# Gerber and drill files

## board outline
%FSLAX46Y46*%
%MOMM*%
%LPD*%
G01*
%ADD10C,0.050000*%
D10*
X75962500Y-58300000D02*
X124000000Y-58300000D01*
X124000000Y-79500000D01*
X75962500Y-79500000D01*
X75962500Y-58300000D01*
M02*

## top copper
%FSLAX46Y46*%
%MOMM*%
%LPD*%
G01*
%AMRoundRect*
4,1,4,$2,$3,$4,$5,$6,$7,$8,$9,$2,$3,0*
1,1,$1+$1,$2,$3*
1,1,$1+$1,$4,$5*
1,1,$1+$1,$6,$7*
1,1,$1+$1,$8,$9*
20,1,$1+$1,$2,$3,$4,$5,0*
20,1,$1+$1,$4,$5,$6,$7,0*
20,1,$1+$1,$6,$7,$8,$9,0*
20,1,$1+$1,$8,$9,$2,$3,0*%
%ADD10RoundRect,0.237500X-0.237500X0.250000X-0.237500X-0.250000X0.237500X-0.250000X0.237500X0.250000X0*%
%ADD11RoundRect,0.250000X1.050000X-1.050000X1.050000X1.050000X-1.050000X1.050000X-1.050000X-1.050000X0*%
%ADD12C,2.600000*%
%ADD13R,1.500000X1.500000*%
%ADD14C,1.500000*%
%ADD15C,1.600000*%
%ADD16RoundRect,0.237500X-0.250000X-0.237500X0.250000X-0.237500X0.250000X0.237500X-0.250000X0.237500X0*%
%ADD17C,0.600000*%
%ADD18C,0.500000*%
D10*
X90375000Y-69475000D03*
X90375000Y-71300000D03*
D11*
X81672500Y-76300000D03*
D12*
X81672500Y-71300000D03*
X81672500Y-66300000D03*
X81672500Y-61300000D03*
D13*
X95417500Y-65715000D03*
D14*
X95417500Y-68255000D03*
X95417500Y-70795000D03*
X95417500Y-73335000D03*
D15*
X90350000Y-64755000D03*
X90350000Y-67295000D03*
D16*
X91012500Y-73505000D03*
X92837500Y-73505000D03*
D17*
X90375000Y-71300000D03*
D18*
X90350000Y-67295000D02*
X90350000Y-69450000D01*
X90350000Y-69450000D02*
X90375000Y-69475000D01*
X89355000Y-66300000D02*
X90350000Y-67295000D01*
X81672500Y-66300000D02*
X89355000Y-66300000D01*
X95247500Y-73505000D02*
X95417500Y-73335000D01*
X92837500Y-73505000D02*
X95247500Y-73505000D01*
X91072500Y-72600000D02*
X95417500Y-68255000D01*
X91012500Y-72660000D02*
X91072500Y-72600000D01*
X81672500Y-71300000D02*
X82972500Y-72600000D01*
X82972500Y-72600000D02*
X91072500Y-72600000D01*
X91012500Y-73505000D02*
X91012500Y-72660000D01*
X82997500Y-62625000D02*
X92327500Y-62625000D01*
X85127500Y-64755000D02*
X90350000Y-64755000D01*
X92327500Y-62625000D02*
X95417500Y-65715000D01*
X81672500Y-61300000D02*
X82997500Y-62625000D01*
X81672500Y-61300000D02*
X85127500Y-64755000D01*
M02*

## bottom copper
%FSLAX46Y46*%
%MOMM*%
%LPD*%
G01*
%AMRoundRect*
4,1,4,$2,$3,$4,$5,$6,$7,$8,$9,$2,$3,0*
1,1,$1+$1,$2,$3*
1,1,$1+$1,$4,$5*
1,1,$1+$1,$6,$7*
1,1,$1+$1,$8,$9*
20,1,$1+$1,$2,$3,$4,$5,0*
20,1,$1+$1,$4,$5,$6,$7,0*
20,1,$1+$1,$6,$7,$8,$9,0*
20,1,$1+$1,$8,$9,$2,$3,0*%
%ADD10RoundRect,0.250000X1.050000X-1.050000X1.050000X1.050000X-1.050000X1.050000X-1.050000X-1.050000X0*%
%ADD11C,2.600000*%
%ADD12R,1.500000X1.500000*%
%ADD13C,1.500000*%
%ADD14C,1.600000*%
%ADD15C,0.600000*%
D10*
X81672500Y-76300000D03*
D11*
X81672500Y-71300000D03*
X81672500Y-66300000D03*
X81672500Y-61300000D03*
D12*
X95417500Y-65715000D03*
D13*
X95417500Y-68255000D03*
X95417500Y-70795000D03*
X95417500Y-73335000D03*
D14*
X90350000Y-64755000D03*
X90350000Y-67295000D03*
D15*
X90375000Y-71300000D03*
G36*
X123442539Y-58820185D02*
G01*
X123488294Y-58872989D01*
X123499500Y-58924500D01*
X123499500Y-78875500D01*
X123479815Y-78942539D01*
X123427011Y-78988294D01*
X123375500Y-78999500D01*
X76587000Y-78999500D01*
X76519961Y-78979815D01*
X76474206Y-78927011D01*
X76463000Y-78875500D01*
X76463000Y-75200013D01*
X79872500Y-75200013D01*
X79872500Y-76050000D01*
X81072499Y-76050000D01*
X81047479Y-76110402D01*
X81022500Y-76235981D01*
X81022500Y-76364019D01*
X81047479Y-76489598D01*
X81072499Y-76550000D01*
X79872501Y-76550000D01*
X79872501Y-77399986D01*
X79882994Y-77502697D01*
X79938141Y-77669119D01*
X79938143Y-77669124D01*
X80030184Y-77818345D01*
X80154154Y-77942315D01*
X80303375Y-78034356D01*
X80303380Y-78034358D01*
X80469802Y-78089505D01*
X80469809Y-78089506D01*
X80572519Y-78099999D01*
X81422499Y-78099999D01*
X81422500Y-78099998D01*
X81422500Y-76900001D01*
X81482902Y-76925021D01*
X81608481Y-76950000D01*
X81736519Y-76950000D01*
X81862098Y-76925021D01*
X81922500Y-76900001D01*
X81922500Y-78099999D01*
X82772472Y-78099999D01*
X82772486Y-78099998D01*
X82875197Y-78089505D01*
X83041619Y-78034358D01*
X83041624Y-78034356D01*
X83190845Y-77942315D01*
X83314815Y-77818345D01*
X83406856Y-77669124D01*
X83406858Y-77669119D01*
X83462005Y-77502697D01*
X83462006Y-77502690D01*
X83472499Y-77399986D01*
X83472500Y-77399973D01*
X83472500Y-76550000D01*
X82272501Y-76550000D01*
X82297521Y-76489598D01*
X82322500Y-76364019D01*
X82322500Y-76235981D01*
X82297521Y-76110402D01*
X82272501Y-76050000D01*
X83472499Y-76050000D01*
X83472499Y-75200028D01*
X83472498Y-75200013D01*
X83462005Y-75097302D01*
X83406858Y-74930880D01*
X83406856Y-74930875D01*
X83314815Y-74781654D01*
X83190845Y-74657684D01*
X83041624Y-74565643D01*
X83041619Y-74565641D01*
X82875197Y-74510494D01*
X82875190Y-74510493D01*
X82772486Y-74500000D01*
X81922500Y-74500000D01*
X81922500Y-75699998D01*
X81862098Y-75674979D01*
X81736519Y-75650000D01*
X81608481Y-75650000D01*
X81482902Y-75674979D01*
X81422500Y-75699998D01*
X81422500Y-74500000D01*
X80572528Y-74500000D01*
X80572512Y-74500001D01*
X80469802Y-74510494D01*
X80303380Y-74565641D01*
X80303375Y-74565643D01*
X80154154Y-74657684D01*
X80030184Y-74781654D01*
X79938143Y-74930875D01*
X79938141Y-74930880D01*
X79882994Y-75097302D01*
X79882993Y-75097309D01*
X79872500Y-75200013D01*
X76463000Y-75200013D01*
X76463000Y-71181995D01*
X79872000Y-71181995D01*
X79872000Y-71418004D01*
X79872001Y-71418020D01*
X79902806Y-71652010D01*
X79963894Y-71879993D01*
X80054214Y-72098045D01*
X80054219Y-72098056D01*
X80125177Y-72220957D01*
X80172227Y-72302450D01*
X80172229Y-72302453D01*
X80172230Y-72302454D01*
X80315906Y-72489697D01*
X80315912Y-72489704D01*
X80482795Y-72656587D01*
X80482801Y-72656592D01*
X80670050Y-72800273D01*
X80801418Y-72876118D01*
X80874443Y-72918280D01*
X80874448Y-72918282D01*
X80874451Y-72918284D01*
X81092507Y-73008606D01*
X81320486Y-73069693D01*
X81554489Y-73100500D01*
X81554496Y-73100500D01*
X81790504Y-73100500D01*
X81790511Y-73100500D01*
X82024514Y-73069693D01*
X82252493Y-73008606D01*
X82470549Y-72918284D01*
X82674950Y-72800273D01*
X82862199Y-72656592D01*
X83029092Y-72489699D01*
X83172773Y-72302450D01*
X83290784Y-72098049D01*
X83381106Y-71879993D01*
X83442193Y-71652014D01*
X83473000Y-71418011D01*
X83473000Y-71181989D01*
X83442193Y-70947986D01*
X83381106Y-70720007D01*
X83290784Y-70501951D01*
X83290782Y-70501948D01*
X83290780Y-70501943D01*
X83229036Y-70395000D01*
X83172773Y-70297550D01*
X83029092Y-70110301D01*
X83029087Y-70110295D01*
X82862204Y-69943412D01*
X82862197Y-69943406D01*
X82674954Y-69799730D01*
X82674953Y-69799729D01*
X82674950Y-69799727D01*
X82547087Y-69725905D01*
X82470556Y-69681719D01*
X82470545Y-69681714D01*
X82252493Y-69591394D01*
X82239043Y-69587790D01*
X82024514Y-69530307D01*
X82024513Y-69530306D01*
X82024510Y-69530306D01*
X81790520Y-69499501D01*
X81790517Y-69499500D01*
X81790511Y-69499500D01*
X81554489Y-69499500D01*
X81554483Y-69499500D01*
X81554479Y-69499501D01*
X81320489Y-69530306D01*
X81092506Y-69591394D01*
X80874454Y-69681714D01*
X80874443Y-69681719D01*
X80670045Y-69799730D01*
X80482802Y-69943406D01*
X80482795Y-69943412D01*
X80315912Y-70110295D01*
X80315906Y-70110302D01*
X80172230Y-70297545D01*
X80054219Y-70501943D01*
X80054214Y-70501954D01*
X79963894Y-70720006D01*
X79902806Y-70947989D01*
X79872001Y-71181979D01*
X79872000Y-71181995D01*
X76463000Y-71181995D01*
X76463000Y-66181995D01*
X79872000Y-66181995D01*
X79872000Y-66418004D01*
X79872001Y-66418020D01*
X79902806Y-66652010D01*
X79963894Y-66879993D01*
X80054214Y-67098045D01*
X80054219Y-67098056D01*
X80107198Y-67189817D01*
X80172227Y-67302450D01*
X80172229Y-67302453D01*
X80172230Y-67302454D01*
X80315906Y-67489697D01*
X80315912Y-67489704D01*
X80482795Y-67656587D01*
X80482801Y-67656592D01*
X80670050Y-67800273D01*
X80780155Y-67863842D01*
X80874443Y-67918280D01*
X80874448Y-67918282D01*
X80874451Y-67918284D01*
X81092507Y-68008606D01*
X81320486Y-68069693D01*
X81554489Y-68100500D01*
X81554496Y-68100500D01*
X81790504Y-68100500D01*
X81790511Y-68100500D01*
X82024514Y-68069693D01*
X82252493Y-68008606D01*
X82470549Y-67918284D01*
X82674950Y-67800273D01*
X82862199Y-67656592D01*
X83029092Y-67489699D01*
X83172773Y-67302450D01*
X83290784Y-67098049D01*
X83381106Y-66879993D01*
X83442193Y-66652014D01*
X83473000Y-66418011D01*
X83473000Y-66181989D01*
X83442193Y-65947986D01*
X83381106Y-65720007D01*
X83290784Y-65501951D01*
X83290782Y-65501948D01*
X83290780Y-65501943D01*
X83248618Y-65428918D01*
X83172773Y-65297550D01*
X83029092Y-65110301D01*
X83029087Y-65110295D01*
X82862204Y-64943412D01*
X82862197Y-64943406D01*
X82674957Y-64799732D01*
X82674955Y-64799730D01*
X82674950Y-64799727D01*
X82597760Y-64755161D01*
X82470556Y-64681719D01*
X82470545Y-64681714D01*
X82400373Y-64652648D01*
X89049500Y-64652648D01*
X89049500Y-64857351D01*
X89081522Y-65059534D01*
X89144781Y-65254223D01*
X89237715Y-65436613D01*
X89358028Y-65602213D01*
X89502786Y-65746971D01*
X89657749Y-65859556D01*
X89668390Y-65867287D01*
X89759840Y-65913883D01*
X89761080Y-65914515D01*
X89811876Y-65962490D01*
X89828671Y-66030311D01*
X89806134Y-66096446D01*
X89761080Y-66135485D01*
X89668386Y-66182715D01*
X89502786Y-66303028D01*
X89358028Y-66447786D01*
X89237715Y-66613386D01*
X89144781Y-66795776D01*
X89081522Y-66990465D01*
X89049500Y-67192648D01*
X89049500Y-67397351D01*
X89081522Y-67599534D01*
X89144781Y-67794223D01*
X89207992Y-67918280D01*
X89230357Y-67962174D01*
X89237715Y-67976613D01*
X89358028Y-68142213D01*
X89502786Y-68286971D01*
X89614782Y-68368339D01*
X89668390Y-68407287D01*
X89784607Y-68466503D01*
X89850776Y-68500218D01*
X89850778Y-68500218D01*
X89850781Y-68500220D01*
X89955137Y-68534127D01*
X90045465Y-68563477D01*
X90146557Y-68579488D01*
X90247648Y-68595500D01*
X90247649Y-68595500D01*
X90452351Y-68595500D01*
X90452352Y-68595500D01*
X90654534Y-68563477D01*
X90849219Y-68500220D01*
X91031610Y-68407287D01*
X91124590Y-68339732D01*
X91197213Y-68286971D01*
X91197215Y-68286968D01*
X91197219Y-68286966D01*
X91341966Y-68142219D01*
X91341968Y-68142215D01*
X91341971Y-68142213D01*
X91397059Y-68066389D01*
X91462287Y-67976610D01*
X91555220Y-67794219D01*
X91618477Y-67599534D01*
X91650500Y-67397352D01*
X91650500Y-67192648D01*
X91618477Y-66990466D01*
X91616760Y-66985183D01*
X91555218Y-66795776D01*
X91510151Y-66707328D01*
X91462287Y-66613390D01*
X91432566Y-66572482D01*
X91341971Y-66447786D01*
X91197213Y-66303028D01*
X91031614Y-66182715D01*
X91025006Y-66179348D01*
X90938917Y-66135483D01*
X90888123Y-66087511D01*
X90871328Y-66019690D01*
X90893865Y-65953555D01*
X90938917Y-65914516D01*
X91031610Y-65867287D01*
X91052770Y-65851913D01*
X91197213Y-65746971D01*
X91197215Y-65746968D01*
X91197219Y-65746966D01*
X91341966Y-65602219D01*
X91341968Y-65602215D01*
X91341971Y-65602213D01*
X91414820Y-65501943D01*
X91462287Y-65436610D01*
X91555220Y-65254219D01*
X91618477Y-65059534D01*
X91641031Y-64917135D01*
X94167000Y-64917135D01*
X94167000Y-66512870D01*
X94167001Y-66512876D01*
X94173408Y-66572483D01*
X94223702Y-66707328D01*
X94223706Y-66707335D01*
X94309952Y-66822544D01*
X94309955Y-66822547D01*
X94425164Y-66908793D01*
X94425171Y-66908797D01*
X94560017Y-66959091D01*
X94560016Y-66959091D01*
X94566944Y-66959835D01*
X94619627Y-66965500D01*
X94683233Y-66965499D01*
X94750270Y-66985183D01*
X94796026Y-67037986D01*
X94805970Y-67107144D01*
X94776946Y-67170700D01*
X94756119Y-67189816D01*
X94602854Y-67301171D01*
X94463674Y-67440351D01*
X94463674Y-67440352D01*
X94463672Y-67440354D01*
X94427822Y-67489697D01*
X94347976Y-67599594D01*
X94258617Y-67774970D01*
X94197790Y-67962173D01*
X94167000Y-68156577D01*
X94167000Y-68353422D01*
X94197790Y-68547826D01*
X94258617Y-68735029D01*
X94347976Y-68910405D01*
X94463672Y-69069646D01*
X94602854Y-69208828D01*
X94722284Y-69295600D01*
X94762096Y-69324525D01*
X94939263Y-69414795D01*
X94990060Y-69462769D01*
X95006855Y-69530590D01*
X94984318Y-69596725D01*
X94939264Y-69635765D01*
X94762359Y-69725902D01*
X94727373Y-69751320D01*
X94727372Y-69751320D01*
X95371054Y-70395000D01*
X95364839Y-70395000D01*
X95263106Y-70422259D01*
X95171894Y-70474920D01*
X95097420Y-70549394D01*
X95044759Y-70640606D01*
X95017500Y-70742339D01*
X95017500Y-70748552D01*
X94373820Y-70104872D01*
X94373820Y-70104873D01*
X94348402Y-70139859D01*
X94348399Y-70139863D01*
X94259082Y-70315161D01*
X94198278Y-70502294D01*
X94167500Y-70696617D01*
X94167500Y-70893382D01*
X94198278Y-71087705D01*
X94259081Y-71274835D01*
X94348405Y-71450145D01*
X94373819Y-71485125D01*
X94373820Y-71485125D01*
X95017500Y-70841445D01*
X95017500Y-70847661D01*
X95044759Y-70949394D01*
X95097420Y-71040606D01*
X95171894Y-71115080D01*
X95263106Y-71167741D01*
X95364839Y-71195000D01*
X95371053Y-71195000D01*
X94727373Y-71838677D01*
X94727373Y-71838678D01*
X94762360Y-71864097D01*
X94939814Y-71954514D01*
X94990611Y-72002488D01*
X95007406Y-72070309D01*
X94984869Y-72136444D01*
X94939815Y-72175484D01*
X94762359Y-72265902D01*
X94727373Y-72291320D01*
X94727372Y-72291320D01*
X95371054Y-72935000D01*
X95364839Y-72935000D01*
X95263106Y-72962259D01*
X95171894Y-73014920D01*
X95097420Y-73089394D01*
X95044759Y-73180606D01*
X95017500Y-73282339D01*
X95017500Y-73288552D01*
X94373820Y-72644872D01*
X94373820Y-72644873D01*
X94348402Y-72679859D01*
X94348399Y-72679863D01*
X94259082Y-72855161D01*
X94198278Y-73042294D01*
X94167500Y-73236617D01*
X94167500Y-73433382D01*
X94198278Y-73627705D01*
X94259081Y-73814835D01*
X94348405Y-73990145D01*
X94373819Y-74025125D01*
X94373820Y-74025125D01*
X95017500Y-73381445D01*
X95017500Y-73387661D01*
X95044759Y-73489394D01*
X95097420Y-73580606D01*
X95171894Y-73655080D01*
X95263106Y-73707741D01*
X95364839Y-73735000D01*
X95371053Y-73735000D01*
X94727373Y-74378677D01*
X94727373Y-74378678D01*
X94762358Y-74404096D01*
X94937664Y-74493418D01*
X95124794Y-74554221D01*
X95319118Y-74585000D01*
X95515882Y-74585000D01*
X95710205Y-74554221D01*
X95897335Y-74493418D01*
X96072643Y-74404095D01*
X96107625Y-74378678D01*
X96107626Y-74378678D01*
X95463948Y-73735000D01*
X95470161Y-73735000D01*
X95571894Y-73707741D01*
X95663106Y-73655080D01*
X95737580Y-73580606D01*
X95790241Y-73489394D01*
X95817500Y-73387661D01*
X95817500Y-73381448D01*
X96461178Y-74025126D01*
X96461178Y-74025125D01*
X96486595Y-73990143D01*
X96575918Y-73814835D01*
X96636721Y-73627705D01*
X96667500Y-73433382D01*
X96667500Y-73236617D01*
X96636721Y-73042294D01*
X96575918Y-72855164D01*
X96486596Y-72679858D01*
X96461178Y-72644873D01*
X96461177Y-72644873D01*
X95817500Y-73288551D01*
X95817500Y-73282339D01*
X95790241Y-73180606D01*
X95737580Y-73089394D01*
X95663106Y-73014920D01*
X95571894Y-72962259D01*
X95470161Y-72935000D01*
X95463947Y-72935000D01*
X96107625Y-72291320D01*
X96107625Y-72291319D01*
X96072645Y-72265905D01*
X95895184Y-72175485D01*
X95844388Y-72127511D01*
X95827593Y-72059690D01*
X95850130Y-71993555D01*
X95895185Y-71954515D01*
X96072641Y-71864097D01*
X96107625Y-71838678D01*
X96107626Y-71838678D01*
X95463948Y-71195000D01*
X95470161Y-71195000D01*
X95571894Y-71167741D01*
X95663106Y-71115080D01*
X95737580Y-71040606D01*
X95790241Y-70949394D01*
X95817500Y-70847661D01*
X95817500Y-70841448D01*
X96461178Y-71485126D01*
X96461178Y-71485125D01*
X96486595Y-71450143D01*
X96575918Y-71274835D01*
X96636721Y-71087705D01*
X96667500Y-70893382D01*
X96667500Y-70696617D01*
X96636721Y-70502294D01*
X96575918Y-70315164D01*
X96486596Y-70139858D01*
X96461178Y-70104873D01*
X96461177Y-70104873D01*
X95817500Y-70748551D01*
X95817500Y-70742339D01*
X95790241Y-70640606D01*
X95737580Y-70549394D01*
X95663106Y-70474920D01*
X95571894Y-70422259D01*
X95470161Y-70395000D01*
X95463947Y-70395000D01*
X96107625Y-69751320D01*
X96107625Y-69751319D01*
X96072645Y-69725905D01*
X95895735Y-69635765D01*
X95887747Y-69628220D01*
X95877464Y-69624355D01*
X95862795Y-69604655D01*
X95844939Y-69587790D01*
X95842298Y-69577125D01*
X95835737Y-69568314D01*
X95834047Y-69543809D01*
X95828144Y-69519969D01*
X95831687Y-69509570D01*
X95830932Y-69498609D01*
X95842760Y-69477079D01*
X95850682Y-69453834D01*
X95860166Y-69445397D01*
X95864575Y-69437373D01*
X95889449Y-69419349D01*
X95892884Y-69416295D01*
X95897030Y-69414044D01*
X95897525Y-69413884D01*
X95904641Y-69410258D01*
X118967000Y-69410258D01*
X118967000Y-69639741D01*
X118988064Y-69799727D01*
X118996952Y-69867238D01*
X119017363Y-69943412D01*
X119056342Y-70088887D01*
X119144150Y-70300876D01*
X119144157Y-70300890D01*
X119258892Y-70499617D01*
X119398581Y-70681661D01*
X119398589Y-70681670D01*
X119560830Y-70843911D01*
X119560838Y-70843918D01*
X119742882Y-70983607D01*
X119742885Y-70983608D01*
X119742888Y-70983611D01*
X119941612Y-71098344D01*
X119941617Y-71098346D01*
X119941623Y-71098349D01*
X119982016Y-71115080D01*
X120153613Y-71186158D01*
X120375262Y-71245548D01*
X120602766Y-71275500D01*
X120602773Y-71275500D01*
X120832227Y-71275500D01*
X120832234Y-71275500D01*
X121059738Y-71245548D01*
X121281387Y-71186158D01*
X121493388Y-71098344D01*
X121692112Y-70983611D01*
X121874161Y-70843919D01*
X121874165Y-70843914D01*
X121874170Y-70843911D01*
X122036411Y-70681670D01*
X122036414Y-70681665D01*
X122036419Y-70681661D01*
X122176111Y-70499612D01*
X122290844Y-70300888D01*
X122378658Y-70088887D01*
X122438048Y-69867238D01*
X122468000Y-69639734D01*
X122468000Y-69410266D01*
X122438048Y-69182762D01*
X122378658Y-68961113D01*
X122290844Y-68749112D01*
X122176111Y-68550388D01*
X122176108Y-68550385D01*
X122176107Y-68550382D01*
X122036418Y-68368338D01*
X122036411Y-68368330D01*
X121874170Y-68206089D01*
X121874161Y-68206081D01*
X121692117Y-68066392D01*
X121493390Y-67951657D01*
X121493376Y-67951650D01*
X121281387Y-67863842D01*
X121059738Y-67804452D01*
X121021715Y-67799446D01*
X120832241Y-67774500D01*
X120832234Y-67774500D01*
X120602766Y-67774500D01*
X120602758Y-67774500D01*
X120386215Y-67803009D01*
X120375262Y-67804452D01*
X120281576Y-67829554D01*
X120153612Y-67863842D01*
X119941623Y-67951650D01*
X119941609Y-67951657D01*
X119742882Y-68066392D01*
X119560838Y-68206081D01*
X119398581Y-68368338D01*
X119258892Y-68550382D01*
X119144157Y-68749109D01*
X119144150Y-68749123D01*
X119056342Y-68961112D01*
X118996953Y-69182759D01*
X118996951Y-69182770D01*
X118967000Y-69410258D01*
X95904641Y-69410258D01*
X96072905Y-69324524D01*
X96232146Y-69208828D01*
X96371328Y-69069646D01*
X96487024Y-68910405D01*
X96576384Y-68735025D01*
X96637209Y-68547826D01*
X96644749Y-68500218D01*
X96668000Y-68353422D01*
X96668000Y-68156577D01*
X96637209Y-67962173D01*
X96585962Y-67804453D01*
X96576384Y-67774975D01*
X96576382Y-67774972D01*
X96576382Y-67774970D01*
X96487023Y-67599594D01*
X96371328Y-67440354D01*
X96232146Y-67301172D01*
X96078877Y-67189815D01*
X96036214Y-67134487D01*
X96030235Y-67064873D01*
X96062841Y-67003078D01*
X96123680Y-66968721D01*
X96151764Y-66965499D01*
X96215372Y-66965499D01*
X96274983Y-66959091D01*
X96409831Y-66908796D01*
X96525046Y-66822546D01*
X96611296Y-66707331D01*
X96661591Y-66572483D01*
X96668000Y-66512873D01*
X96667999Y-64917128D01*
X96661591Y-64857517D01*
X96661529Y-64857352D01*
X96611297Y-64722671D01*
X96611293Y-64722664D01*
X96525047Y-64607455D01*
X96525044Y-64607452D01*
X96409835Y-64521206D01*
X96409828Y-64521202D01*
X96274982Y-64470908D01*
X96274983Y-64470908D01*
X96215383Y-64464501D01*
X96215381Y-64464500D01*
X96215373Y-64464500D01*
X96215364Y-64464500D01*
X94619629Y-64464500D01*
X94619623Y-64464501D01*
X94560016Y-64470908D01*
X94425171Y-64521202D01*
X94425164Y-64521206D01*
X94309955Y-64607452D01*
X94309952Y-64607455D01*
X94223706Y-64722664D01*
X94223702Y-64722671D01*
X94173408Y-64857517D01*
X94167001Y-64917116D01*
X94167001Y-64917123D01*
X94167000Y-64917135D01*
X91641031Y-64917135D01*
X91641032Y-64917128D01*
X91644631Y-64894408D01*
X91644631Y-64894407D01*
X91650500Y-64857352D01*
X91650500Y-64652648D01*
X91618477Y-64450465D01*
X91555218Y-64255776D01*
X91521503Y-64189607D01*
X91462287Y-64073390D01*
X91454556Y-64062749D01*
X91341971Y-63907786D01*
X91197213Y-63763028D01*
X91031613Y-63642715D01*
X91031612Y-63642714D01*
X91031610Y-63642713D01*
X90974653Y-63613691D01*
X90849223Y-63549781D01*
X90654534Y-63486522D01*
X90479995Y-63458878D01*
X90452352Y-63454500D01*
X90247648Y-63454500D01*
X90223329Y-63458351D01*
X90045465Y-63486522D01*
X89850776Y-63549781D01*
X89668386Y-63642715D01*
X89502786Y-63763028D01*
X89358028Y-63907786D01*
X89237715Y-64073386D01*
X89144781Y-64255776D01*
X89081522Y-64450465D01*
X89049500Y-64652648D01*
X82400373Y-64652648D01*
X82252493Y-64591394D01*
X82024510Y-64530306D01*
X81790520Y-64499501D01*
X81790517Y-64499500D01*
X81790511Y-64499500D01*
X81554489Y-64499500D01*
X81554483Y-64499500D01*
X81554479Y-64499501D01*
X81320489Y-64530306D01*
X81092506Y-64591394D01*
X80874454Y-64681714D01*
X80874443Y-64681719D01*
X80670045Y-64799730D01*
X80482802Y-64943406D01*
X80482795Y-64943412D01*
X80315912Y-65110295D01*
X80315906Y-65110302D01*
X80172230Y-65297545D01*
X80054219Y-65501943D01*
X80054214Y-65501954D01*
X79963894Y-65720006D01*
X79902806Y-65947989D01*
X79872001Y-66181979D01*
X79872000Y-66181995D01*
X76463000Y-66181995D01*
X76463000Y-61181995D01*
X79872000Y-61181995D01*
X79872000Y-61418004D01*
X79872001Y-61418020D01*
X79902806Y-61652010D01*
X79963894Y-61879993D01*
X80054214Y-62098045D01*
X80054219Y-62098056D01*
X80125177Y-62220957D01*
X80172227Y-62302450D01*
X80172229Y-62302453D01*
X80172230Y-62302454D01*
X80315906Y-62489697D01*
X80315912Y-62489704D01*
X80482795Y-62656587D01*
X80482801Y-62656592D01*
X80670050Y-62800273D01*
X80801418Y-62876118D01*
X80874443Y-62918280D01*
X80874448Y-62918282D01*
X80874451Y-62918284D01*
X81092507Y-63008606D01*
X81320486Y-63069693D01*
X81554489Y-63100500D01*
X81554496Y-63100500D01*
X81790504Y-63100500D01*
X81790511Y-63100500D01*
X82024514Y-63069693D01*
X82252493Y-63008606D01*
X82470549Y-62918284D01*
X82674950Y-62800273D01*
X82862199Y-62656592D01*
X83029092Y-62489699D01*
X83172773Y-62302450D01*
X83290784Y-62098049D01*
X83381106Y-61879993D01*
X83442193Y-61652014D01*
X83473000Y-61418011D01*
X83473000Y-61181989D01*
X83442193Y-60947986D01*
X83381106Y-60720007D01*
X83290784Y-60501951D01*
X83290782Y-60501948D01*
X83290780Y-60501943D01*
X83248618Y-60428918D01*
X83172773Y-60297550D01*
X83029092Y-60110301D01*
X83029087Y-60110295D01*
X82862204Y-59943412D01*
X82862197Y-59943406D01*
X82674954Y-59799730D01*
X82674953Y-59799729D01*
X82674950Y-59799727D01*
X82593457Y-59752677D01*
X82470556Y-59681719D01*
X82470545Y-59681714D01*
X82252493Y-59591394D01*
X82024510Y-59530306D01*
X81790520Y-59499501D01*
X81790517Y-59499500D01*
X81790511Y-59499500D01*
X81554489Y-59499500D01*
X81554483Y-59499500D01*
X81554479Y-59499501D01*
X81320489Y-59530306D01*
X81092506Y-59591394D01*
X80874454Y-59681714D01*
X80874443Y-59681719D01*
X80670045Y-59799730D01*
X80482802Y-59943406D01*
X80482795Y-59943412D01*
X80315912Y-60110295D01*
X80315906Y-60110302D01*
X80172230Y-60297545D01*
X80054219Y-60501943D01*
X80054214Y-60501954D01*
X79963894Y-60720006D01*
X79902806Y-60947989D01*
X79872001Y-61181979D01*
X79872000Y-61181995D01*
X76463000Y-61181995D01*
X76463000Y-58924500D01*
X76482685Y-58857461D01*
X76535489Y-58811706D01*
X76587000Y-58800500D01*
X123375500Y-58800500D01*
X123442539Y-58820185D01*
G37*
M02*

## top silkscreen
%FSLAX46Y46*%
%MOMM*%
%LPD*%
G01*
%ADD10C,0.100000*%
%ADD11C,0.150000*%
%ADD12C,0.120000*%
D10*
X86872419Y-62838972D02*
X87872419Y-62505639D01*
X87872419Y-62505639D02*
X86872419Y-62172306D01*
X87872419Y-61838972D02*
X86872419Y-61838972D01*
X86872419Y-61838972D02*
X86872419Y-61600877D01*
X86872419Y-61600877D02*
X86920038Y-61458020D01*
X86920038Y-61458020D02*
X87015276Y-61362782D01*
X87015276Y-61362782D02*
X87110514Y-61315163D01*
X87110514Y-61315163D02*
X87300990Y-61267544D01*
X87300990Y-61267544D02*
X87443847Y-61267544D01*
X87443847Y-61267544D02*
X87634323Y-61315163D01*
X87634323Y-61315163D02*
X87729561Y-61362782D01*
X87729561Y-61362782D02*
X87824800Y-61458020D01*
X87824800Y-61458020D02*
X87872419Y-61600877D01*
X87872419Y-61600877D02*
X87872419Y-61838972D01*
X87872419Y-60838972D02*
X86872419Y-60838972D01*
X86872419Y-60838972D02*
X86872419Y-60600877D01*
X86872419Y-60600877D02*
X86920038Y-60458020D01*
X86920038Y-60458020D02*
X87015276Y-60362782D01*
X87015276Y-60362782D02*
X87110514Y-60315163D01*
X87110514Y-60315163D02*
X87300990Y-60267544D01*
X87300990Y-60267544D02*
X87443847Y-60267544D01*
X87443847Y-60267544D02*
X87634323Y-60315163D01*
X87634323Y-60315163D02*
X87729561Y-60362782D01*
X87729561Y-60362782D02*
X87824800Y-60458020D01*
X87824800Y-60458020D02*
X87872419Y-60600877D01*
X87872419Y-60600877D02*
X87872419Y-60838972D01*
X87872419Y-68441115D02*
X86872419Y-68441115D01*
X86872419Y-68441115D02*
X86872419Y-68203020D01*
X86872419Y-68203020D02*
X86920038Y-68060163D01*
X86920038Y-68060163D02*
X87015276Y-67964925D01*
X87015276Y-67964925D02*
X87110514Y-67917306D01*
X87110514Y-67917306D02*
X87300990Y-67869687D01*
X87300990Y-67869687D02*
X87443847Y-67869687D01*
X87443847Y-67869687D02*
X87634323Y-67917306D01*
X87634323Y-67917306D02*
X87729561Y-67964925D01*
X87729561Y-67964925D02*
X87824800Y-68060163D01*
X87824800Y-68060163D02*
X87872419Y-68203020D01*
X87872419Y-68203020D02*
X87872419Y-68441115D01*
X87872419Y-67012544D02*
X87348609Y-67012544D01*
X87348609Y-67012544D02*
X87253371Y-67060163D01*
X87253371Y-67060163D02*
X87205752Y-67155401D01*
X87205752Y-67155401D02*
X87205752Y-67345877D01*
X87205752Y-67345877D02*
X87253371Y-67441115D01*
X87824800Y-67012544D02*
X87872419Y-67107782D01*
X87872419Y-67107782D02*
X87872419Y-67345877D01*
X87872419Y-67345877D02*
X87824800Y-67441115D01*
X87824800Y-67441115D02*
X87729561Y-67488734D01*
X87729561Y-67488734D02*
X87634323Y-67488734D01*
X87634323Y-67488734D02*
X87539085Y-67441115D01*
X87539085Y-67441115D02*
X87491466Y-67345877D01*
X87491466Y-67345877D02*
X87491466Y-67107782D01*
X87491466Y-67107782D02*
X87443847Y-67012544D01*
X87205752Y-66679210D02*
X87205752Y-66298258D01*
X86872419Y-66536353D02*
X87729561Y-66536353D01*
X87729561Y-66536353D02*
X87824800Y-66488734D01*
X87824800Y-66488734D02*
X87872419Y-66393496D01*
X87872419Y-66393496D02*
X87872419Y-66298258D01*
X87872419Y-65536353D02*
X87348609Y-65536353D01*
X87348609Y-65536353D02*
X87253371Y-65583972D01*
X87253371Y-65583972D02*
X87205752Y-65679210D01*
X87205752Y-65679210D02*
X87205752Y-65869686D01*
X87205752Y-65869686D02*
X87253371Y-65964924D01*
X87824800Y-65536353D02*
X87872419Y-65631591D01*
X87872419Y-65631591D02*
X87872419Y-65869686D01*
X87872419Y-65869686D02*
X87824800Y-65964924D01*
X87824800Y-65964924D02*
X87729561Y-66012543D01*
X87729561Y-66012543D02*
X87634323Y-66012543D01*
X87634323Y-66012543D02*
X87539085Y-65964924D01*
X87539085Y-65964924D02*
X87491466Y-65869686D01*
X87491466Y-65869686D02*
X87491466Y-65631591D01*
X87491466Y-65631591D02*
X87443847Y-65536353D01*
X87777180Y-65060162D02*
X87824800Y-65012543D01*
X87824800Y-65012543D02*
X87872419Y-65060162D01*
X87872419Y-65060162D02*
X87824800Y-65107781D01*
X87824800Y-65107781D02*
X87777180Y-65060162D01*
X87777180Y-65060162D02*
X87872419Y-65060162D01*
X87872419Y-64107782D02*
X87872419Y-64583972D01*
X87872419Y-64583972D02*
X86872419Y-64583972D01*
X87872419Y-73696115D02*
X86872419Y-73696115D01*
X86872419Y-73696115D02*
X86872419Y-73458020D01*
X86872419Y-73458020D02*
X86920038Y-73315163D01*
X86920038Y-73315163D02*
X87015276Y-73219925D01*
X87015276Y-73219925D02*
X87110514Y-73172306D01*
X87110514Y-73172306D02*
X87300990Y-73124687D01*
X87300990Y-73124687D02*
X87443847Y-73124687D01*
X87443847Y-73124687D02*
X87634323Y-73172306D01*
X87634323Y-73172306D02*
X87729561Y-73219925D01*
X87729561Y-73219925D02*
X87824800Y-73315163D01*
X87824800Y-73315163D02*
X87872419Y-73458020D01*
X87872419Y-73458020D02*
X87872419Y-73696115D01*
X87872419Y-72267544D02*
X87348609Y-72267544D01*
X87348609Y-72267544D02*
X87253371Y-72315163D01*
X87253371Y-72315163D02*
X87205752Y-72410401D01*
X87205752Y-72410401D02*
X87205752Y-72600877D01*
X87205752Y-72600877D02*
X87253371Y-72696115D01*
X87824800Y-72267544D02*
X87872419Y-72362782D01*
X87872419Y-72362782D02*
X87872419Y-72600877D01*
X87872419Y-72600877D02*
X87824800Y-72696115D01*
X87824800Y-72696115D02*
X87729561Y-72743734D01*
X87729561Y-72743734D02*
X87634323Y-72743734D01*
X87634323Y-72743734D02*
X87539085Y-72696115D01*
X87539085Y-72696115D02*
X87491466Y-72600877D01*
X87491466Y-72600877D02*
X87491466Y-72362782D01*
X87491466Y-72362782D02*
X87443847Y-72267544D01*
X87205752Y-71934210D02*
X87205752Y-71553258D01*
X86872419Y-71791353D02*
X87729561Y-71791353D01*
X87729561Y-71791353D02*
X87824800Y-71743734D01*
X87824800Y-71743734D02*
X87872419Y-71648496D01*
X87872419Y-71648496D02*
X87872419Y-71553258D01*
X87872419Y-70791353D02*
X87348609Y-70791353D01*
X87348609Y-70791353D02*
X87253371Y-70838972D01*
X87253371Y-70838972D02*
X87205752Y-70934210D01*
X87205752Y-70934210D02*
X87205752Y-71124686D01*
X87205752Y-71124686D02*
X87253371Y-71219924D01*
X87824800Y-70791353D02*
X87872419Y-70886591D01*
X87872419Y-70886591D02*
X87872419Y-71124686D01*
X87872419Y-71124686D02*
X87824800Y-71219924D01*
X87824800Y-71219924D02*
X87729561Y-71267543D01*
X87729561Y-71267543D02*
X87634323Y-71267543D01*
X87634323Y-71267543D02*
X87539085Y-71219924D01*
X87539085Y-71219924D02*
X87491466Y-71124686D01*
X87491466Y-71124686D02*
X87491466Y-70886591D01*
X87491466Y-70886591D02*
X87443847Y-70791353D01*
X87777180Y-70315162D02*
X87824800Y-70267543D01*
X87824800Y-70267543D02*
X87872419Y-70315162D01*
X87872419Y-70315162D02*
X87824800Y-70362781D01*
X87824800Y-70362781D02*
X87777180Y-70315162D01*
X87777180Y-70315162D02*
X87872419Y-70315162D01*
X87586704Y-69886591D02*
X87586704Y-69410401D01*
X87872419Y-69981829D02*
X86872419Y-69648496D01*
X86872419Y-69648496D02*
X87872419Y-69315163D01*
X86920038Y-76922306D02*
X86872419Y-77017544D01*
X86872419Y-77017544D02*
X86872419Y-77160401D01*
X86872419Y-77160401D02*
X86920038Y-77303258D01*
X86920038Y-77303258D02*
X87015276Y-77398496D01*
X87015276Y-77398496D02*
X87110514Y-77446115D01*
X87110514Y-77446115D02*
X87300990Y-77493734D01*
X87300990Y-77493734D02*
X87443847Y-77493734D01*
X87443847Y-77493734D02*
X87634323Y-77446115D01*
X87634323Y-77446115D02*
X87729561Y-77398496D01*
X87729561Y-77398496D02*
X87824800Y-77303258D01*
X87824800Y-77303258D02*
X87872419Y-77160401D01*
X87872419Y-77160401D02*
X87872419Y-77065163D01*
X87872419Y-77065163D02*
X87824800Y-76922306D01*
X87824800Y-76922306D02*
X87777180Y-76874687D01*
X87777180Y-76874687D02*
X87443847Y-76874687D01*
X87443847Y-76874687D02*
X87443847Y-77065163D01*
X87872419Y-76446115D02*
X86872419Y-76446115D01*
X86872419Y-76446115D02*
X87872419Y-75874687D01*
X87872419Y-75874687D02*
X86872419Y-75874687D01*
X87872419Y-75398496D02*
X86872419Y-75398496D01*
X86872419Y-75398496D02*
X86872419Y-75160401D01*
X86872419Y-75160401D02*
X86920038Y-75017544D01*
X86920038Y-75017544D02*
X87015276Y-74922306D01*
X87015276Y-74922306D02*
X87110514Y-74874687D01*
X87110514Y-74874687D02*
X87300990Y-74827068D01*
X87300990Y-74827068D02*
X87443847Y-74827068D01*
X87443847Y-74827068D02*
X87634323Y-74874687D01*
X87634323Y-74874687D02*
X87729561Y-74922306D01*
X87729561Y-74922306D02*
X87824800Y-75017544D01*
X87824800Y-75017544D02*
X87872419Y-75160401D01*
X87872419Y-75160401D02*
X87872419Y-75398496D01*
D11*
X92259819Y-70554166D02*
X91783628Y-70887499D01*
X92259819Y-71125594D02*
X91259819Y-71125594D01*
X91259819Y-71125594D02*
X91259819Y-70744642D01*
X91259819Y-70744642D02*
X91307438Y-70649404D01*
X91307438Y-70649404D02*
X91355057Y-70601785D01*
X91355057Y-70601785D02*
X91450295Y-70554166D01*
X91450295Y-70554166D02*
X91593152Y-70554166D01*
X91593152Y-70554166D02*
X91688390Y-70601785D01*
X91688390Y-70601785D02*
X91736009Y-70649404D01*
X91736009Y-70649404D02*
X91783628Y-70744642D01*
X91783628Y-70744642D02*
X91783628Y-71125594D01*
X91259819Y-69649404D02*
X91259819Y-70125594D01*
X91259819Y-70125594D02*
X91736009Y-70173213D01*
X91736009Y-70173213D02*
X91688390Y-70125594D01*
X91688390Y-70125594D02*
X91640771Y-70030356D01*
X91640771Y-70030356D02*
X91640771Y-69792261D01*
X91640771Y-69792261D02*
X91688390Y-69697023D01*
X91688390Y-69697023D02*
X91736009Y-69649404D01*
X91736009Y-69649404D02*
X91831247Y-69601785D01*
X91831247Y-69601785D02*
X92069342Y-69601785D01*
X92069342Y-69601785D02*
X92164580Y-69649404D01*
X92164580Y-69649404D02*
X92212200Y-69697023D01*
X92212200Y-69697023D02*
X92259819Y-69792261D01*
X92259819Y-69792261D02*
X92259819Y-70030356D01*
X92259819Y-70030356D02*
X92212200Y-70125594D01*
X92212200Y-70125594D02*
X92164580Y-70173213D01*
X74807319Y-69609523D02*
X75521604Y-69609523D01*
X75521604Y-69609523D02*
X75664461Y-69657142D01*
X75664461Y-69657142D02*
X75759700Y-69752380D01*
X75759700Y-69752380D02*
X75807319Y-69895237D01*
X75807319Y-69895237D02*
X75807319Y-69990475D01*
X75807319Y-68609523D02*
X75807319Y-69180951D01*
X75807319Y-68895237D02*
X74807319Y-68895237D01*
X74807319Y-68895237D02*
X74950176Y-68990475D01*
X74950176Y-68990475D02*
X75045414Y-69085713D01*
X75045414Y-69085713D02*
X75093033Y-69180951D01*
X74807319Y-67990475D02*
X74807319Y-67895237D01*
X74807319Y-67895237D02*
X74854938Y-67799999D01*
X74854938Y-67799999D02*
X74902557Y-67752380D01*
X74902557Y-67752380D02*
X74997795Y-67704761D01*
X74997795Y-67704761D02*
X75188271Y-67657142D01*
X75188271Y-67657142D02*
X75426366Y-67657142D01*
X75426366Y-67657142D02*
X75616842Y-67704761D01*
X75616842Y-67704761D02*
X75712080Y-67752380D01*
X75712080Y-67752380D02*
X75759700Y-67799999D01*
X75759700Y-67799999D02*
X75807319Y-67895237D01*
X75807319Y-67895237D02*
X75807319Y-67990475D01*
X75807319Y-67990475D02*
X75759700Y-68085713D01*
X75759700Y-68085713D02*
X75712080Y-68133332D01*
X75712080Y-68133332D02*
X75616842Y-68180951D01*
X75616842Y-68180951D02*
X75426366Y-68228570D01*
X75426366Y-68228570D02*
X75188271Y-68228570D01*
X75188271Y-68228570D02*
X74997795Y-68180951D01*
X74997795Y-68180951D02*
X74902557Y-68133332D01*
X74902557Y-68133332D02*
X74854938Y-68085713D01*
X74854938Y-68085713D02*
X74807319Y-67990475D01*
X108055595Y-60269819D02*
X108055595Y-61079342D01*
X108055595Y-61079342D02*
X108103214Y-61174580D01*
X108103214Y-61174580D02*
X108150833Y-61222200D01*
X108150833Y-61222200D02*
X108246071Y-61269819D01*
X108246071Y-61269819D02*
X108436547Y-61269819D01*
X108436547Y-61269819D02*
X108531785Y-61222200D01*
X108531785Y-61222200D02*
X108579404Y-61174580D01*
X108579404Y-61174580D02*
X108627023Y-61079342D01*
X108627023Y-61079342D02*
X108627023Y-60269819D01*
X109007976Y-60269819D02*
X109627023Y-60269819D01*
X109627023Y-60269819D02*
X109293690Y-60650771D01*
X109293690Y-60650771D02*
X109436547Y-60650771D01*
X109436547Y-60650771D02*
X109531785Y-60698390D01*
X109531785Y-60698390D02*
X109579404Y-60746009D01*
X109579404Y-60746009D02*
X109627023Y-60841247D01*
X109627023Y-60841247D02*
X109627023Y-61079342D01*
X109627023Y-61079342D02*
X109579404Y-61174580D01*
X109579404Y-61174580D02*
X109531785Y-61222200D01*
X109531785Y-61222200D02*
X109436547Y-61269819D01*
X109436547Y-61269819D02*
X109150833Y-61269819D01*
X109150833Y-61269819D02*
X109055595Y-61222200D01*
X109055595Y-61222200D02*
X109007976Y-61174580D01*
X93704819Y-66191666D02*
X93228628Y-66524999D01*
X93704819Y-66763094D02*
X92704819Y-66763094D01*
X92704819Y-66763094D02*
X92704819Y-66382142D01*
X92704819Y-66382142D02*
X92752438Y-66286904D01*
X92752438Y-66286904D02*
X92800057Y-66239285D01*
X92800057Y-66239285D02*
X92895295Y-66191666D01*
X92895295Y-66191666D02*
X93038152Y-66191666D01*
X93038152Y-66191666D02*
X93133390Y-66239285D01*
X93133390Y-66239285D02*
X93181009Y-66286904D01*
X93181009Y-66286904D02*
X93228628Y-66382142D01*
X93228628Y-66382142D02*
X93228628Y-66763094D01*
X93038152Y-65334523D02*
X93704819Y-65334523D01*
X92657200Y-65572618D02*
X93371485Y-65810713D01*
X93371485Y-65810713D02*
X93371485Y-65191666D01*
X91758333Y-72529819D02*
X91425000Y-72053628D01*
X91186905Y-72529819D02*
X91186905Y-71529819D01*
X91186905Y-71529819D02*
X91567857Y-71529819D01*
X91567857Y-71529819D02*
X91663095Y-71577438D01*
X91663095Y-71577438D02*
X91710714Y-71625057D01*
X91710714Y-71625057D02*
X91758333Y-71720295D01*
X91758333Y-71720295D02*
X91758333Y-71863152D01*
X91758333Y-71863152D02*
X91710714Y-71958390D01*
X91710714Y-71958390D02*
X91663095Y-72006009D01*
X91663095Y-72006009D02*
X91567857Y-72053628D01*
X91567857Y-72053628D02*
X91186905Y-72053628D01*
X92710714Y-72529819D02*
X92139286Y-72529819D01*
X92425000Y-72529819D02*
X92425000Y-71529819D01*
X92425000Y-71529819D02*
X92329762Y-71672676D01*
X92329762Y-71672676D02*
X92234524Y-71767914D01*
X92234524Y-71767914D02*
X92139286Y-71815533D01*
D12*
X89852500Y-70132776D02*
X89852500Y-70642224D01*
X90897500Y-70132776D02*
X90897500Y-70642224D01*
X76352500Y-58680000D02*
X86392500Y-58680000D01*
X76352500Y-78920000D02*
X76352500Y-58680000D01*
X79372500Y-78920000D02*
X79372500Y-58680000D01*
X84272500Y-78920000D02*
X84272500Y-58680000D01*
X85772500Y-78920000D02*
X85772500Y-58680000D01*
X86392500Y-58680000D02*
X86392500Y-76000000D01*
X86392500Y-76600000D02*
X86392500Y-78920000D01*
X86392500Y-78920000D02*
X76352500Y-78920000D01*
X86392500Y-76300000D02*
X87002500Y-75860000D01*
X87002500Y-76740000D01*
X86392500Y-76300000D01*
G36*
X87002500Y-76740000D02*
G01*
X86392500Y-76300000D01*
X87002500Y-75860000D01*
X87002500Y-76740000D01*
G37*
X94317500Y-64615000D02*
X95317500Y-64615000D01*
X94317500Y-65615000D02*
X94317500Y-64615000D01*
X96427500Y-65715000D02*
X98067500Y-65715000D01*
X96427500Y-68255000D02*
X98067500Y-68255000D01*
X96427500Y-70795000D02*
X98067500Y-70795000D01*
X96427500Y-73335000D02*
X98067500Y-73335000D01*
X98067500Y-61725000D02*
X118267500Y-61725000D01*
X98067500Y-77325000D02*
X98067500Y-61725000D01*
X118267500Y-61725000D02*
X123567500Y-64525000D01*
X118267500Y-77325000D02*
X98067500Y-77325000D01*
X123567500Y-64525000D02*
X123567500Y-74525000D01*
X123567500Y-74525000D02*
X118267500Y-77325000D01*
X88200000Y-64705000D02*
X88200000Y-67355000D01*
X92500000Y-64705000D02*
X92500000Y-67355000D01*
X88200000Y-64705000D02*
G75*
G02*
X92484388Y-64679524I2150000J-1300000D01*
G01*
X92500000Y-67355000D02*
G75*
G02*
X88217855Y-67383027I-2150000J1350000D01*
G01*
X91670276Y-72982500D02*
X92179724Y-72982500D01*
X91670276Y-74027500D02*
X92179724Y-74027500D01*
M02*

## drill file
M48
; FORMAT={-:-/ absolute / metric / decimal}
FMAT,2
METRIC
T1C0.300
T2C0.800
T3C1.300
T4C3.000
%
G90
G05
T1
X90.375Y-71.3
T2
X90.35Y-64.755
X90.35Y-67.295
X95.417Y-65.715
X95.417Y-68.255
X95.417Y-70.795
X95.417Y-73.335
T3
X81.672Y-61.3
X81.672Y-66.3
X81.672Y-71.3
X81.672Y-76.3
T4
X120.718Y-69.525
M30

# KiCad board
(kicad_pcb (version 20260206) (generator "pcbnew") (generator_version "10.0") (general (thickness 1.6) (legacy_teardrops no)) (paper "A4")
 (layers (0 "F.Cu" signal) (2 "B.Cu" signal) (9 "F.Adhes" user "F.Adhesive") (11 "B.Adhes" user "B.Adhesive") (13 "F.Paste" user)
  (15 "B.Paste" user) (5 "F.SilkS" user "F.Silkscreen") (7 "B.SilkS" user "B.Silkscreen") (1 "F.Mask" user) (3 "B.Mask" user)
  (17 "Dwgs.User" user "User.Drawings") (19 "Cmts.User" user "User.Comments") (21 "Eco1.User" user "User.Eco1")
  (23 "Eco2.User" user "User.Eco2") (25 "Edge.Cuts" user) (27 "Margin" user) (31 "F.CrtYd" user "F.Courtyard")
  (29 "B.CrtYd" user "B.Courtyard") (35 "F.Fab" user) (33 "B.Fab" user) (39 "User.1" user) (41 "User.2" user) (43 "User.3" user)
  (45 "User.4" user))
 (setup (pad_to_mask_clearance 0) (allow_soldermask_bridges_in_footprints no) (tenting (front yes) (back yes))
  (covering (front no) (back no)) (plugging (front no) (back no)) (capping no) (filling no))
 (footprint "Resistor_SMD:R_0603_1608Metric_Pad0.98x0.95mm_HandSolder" (layer "F.Cu") (at 90.375 70.3875 -90)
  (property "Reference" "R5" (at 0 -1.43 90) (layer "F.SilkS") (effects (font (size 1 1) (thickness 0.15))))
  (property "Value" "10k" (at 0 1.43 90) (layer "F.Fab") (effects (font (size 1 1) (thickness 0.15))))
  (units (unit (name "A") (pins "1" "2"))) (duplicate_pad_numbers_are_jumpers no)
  (fp_line (start -0.254724 0.5225) (end 0.254724 0.5225) (stroke (width 0.12) (type solid)) (layer "F.SilkS"))
  (fp_line (start -0.254724 -0.5225) (end 0.254724 -0.5225) (stroke (width 0.12) (type solid)) (layer "F.SilkS"))
  (pad "1" smd roundrect (at -0.9125 0 270) (size 0.975 0.95) (layers "F.Cu" "F.Mask" "F.Paste") (roundrect_rratio 0.25)
   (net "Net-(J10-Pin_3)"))
  (pad "2" smd roundrect (at 0.9125 0 270) (size 0.975 0.95) (layers "F.Cu" "F.Mask" "F.Paste") (roundrect_rratio 0.25) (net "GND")))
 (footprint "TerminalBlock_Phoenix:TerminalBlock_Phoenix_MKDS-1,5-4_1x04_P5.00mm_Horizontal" (layer "F.Cu") (at 81.6725 76.3 90)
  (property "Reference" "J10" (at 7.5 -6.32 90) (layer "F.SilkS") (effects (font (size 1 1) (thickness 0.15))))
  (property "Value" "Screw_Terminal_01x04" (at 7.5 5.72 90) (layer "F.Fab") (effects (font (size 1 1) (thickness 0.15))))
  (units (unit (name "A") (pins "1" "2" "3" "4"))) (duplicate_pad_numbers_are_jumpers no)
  (fp_line (start 17.62 -5.32) (end 17.62 4.72) (stroke (width 0.12) (type solid)) (layer "F.SilkS"))
  (fp_line (start -2.62 -5.32) (end 17.62 -5.32) (stroke (width 0.12) (type solid)) (layer "F.SilkS"))
  (fp_line (start -2.62 -2.3) (end 17.62 -2.3) (stroke (width 0.12) (type solid)) (layer "F.SilkS"))
  (fp_line (start -2.62 2.6) (end 17.62 2.6) (stroke (width 0.12) (type solid)) (layer "F.SilkS"))
  (fp_line (start -2.62 4.1) (end 17.62 4.1) (stroke (width 0.12) (type solid)) (layer "F.SilkS"))
  (fp_line (start 17.62 4.72) (end 0.3 4.72) (stroke (width 0.12) (type solid)) (layer "F.SilkS"))
  (fp_line (start -0.3 4.72) (end -2.62 4.72) (stroke (width 0.12) (type solid)) (layer "F.SilkS"))
  (fp_line (start -2.62 4.72) (end -2.62 -5.32) (stroke (width 0.12) (type solid)) (layer "F.SilkS"))
  (fp_poly (pts (xy 0 4.72) (xy 0.44 5.33) (xy -0.44 5.33)) (stroke (width 0.12) (type solid)) (fill yes) (layer "F.SilkS"))
  (pad "1" thru_hole roundrect (at 0 0 90) (size 2.6 2.6) (drill 1.3) (layers "*.Cu" "*.Mask") (remove_unused_layers no)
   (roundrect_rratio 0.096154) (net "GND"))
  (pad "2" thru_hole circle (at 5 0 90) (size 2.6 2.6) (drill 1.3) (layers "*.Cu" "*.Mask") (remove_unused_layers no)
   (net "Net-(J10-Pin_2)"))
  (pad "3" thru_hole circle (at 10 0 90) (size 2.6 2.6) (drill 1.3) (layers "*.Cu" "*.Mask") (remove_unused_layers no)
   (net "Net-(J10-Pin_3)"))
  (pad "4" thru_hole circle (at 15 0 90) (size 2.6 2.6) (drill 1.3) (layers "*.Cu" "*.Mask") (remove_unused_layers no) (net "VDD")))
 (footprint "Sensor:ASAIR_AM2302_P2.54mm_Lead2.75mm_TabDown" (layer "F.Cu") (at 95.4175 65.715)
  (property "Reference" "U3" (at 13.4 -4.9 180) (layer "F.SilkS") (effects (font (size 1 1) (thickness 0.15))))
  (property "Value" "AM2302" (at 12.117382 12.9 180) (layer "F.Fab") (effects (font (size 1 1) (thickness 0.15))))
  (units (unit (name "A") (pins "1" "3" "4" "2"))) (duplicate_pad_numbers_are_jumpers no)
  (fp_line (start -1.1 -1.1) (end -0.1 -1.1) (stroke (width 0.12) (type default)) (layer "F.SilkS"))
  (fp_line (start -1.1 -0.1) (end -1.1 -1.1) (stroke (width 0.12) (type default)) (layer "F.SilkS"))
  (fp_line (start 1.01 0) (end 2.65 0) (stroke (width 0.12) (type default)) (layer "F.SilkS"))
  (fp_line (start 1.01 2.54) (end 2.65 2.54) (stroke (width 0.12) (type default)) (layer "F.SilkS"))
  (fp_line (start 1.01 5.08) (end 2.65 5.08) (stroke (width 0.12) (type default)) (layer "F.SilkS"))
  (fp_line (start 1.01 7.62) (end 2.65 7.62) (stroke (width 0.12) (type default)) (layer "F.SilkS"))
  (fp_line (start 2.65 -3.99) (end 22.85 -3.99) (stroke (width 0.12) (type solid)) (layer "F.SilkS"))
  (fp_line (start 2.65 11.61) (end 2.65 -3.99) (stroke (width 0.12) (type solid)) (layer "F.SilkS"))
  (fp_line (start 22.85 -3.99) (end 28.15 -1.19) (stroke (width 0.12) (type default)) (layer "F.SilkS"))
  (fp_line (start 22.85 11.61) (end 2.65 11.61) (stroke (width 0.12) (type solid)) (layer "F.SilkS"))
  (fp_line (start 28.15 -1.19) (end 28.15 8.81) (stroke (width 0.12) (type solid)) (layer "F.SilkS"))
  (fp_line (start 28.15 8.81) (end 22.85 11.61) (stroke (width 0.12) (type default)) (layer "F.SilkS"))
  (pad "" np_thru_hole circle (at 25.3 3.81) (size 3 3) (drill 3) (layers "*.Cu" "*.Mask"))
  (pad "1" thru_hole rect (at 0 0) (size 1.5 1.5) (drill 0.8) (layers "*.Cu" "*.Mask") (remove_unused_layers no) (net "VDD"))
  (pad "2" thru_hole circle (at 0 2.54) (size 1.5 1.5) (drill 0.8) (layers "*.Cu" "*.Mask") (remove_unused_layers no)
   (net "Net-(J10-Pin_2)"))
  (pad "3" thru_hole circle (at 0 5.08) (size 1.5 1.5) (drill 0.8) (layers "*.Cu" "*.Mask") (remove_unused_layers no) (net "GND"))
  (pad "4" thru_hole circle (at 0 7.62) (size 1.5 1.5) (drill 0.8) (layers "*.Cu" "*.Mask") (remove_unused_layers no) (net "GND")))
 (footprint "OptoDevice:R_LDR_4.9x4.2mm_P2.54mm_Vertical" (layer "F.Cu") (at 90.35 64.755 -90)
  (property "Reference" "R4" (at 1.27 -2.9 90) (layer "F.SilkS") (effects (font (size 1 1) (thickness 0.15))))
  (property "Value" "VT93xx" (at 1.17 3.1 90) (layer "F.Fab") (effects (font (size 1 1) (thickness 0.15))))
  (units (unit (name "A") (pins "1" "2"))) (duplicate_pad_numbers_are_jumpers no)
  (fp_line (start -0.05 2.15) (end 2.6 2.15) (stroke (width 0.12) (type solid)) (layer "F.SilkS"))
  (fp_line (start -0.05 -2.15) (end 2.6 -2.15) (stroke (width 0.12) (type solid)) (layer "F.SilkS"))
  (fp_arc (start -0.05 2.15) (mid -1.262424 0.01494) (end -0.075476 -2.134388) (stroke (width 0.12) (type solid)) (layer "F.SilkS"))
  (fp_arc (start 2.6 -2.15) (mid 3.788646 -0.016616) (end 2.628027 2.132145) (stroke (width 0.12) (type solid)) (layer "F.SilkS"))
  (pad "1" thru_hole circle (at 0 0 270) (size 1.6 1.6) (drill 0.8) (layers "*.Cu" "*.Mask") (remove_unused_layers no) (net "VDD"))
  (pad "2" thru_hole circle (at 2.54 0 270) (size 1.6 1.6) (drill 0.8) (layers "*.Cu" "*.Mask") (remove_unused_layers no)
   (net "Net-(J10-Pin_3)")))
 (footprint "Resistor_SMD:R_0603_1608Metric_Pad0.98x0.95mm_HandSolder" (layer "F.Cu") (at 91.925 73.505)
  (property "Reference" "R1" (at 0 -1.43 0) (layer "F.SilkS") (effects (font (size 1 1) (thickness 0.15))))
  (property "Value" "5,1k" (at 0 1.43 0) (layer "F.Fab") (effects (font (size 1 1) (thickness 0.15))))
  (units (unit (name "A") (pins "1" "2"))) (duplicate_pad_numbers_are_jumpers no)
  (fp_line (start -0.254724 -0.5225) (end 0.254724 -0.5225) (stroke (width 0.12) (type solid)) (layer "F.SilkS"))
  (fp_line (start -0.254724 0.5225) (end 0.254724 0.5225) (stroke (width 0.12) (type solid)) (layer "F.SilkS"))
  (pad "1" smd roundrect (at -0.9125 0) (size 0.975 0.95) (layers "F.Cu" "F.Mask" "F.Paste") (roundrect_rratio 0.25) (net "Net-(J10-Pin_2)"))
  (pad "2" smd roundrect (at 0.9125 0) (size 0.975 0.95) (layers "F.Cu" "F.Mask" "F.Paste") (roundrect_rratio 0.25) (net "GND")))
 (gr_rect (start 75.9625 58.3) (end 124 79.5) (stroke (width 0.05) (type default)) (fill no) (layer "Edge.Cuts"))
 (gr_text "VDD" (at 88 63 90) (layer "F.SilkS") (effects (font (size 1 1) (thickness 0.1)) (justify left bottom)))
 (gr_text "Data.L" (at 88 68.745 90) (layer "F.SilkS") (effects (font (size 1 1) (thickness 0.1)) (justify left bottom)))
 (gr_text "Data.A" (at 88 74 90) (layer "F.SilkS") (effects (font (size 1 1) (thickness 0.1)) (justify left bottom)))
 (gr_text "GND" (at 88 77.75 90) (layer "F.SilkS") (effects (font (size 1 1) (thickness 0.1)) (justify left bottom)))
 (segment (start 90.35 67.295) (end 90.35 69.45) (width 0.5) (layer "F.Cu") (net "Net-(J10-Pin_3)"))
 (segment (start 90.35 69.45) (end 90.375 69.475) (width 0.5) (layer "F.Cu") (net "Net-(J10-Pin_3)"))
 (segment (start 89.355 66.3) (end 90.35 67.295) (width 0.5) (layer "F.Cu") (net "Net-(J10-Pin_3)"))
 (segment (start 81.6725 66.3) (end 89.355 66.3) (width 0.5) (layer "F.Cu") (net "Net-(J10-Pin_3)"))
 (segment (start 95.2475 73.505) (end 95.4175 73.335) (width 0.5) (layer "F.Cu") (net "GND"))
 (segment (start 92.8375 73.505) (end 95.2475 73.505) (width 0.5) (layer "F.Cu") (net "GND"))
 (via (at 90.375 71.3) (size 0.6) (drill 0.3) (layers "F.Cu" "B.Cu") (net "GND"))
 (segment (start 91.0725 72.6) (end 95.4175 68.255) (width 0.5) (layer "F.Cu") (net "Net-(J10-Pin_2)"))
 (segment (start 91.0125 72.66) (end 91.0725 72.6) (width 0.5) (layer "F.Cu") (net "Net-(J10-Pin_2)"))
 (segment (start 81.6725 71.3) (end 82.9725 72.6) (width 0.5) (layer "F.Cu") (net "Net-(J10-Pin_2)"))
 (segment (start 82.9725 72.6) (end 91.0725 72.6) (width 0.5) (layer "F.Cu") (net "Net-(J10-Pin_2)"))
 (segment (start 91.0125 73.505) (end 91.0125 72.66) (width 0.5) (layer "F.Cu") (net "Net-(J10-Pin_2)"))
 (segment (start 82.9975 62.625) (end 92.3275 62.625) (width 0.5) (layer "F.Cu") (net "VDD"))
 (segment (start 85.1275 64.755) (end 90.35 64.755) (width 0.5) (layer "F.Cu") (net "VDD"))
 (segment (start 92.3275 62.625) (end 95.4175 65.715) (width 0.5) (layer "F.Cu") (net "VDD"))
 (segment (start 81.6725 61.3) (end 82.9975 62.625) (width 0.5) (layer "F.Cu") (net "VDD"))
 (segment (start 81.6725 61.3) (end 85.1275 64.755) (width 0.5) (layer "F.Cu") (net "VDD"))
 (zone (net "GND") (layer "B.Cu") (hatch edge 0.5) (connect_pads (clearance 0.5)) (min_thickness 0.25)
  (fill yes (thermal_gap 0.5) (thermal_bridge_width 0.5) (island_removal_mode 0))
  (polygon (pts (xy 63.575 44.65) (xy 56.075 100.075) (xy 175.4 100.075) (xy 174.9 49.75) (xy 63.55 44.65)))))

